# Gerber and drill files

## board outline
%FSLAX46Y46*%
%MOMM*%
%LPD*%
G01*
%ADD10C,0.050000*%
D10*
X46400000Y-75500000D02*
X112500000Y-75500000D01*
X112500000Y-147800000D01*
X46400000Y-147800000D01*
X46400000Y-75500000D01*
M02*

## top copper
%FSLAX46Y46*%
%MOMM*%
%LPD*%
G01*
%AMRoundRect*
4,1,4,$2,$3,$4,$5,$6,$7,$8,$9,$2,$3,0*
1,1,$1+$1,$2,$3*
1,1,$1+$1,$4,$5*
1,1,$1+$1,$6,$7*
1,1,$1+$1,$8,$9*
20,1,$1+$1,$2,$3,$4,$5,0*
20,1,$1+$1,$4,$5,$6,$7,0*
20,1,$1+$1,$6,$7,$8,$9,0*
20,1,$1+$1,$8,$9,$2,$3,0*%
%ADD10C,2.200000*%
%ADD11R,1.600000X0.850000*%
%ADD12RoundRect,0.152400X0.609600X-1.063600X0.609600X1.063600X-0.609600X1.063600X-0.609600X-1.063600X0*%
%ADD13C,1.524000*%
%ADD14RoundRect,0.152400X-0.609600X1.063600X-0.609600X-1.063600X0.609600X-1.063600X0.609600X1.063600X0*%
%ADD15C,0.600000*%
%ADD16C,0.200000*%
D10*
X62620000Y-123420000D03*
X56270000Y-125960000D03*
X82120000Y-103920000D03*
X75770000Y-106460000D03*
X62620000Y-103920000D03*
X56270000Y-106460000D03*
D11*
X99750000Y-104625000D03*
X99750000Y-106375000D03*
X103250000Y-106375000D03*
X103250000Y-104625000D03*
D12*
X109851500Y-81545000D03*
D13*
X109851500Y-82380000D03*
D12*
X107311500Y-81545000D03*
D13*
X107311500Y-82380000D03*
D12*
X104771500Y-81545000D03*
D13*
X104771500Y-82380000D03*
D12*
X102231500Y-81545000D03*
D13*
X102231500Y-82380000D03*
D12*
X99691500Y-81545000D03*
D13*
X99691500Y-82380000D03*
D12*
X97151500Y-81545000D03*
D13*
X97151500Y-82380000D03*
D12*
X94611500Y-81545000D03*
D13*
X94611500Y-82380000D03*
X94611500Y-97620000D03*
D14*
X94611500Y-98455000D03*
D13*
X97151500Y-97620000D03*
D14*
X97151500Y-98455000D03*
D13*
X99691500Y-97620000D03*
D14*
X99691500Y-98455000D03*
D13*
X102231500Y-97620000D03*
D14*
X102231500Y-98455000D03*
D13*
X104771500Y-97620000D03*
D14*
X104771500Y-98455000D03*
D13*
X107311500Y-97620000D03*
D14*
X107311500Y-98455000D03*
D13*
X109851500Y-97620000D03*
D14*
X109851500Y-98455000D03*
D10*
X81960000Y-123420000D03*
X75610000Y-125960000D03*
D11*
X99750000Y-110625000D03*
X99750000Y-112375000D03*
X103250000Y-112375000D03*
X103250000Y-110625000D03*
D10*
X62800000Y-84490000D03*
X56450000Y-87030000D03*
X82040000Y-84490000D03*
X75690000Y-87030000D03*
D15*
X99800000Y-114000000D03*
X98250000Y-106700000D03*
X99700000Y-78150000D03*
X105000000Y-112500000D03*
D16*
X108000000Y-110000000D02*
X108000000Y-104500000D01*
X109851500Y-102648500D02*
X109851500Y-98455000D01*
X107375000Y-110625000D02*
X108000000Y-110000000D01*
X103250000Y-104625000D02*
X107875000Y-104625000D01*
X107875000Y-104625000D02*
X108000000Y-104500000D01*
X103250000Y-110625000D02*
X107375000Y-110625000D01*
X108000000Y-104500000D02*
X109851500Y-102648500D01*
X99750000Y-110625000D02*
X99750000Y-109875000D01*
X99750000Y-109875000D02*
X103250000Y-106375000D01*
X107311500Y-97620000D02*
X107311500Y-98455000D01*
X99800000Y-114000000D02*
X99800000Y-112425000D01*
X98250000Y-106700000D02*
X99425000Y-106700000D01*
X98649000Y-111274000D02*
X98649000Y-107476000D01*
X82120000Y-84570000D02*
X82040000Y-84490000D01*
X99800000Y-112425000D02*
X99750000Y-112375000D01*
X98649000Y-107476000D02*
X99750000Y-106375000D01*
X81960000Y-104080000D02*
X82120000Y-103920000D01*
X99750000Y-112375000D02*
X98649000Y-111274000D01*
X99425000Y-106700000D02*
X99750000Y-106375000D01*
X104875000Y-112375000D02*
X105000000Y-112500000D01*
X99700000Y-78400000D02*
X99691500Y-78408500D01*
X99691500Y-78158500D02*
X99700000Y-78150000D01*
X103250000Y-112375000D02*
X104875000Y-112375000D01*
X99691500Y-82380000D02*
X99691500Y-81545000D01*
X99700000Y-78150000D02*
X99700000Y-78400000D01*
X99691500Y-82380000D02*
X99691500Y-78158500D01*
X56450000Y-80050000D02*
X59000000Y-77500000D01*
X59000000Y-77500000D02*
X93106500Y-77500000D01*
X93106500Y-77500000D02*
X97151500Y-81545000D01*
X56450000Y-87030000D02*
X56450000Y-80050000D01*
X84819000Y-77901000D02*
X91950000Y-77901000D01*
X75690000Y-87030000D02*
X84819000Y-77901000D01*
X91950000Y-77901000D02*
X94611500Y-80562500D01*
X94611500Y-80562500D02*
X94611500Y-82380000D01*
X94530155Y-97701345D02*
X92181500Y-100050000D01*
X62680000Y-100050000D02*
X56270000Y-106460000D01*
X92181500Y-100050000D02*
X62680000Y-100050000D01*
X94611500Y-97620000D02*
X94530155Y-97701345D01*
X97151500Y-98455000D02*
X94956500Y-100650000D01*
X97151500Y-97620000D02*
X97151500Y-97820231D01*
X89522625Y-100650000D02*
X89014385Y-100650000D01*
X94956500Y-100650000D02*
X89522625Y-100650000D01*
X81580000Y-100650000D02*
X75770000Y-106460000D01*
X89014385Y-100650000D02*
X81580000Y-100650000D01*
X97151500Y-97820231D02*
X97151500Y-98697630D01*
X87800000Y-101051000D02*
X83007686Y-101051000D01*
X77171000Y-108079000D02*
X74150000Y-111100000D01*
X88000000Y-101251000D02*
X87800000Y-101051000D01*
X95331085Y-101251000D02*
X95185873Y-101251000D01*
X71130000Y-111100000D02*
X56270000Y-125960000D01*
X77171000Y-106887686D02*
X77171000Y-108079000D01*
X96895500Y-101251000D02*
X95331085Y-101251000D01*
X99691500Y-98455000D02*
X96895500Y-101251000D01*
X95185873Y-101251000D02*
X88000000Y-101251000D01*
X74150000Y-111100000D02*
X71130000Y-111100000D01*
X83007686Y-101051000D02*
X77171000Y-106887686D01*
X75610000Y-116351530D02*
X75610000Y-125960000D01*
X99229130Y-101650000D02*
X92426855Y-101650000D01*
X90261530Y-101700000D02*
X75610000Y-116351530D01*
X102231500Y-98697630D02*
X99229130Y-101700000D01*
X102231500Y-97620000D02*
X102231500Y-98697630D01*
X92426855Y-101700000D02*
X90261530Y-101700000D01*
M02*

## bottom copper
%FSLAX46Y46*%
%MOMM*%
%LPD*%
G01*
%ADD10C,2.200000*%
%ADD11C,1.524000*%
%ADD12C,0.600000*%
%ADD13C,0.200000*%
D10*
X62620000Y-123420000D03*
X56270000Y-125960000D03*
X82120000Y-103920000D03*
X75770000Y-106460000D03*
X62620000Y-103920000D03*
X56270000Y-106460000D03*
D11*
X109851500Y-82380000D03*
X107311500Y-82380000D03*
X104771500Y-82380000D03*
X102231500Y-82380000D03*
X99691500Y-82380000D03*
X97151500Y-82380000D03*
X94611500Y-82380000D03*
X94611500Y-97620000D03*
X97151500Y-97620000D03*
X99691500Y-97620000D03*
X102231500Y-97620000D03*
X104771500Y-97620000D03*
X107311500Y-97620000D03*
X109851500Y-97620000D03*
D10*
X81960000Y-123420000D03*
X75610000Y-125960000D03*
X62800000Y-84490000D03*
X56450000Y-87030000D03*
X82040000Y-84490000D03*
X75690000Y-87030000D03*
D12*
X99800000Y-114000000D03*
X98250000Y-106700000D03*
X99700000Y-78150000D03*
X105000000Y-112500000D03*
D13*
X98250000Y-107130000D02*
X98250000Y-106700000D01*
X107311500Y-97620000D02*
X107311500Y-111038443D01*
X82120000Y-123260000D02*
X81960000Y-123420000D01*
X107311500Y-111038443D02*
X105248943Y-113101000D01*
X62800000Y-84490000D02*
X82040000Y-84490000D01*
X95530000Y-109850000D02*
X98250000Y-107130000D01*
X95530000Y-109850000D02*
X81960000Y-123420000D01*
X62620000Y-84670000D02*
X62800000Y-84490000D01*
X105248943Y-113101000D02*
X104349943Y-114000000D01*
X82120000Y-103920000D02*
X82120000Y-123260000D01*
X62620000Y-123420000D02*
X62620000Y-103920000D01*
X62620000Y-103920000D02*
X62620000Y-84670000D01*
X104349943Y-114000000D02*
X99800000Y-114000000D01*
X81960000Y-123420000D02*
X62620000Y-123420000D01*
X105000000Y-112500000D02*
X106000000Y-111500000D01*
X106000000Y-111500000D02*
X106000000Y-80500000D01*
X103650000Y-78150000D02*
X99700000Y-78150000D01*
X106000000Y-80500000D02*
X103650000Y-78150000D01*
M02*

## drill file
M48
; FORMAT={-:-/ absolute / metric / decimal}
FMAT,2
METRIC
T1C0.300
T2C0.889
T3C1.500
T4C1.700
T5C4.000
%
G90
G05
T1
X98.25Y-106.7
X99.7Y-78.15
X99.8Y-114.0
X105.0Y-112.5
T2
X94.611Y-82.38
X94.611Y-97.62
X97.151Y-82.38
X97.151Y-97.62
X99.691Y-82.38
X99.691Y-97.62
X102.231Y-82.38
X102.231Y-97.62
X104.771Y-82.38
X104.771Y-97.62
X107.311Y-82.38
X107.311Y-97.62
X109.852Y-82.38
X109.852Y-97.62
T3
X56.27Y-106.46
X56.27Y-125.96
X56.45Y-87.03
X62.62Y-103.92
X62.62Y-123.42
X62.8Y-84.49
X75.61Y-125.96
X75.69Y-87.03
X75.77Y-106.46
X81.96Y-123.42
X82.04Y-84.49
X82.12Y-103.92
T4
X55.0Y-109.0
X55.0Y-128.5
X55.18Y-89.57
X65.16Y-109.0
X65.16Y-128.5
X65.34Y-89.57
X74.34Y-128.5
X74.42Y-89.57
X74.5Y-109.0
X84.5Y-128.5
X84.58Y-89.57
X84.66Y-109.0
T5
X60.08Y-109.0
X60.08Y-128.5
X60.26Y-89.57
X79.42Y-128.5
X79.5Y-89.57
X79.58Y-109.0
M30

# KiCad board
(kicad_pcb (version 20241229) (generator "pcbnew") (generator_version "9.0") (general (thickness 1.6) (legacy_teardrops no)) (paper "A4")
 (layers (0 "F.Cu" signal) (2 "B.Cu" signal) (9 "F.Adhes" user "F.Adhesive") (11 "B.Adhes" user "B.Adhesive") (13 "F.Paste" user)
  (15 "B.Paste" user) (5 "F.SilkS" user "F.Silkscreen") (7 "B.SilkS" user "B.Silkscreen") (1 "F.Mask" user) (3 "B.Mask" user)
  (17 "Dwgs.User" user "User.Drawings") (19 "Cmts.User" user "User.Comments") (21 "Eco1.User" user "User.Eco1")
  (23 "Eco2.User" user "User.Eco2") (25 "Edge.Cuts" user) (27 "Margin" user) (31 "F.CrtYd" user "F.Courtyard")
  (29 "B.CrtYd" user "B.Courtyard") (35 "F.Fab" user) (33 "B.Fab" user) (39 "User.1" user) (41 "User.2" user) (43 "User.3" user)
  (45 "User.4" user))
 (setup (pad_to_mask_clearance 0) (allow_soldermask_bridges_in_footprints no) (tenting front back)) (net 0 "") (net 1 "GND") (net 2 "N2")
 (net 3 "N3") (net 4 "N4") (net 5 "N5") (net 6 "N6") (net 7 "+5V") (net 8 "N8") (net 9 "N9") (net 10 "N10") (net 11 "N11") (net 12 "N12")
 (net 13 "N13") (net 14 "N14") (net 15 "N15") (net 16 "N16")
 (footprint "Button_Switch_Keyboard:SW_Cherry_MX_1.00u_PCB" (layer "F.Cu") (at 62.62 123.42)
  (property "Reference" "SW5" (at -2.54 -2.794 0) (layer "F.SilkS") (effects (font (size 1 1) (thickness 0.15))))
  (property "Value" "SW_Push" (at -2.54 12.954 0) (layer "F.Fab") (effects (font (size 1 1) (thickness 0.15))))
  (pad "" np_thru_hole circle (at -7.62 5.08) (size 1.7 1.7) (drill 1.7) (layers "*.Cu" "*.Mask"))
  (pad "" np_thru_hole circle (at -2.54 5.08) (size 4 4) (drill 4) (layers "*.Cu" "*.Mask"))
  (pad "" np_thru_hole circle (at 2.54 5.08) (size 1.7 1.7) (drill 1.7) (layers "*.Cu" "*.Mask"))
  (pad "1" thru_hole circle (at 0 0) (size 2.2 2.2) (drill 1.5) (layers "*.Cu" "*.Mask") (remove_unused_layers no) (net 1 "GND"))
  (pad "2" thru_hole circle (at -6.35 2.54) (size 2.2 2.2) (drill 1.5) (layers "*.Cu" "*.Mask") (remove_unused_layers no) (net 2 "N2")))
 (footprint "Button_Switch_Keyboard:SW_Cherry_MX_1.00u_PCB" (layer "F.Cu") (at 82.12 103.92)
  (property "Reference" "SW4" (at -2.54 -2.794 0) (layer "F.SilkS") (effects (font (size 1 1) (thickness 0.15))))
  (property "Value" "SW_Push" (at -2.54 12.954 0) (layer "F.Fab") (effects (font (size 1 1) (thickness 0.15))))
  (pad "" np_thru_hole circle (at -7.62 5.08) (size 1.7 1.7) (drill 1.7) (layers "*.Cu" "*.Mask"))
  (pad "" np_thru_hole circle (at -2.54 5.08) (size 4 4) (drill 4) (layers "*.Cu" "*.Mask"))
  (pad "" np_thru_hole circle (at 2.54 5.08) (size 1.7 1.7) (drill 1.7) (layers "*.Cu" "*.Mask"))
  (pad "1" thru_hole circle (at 0 0) (size 2.2 2.2) (drill 1.5) (layers "*.Cu" "*.Mask") (remove_unused_layers no) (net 1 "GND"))
  (pad "2" thru_hole circle (at -6.35 2.54) (size 2.2 2.2) (drill 1.5) (layers "*.Cu" "*.Mask") (remove_unused_layers no) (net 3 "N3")))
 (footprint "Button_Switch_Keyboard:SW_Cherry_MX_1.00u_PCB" (layer "F.Cu") (at 62.62 103.92)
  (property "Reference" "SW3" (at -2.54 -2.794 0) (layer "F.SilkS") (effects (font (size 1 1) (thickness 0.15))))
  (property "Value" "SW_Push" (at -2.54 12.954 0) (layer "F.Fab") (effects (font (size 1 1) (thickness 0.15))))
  (pad "" np_thru_hole circle (at -7.62 5.08) (size 1.7 1.7) (drill 1.7) (layers "*.Cu" "*.Mask"))
  (pad "" np_thru_hole circle (at -2.54 5.08) (size 4 4) (drill 4) (layers "*.Cu" "*.Mask"))
  (pad "" np_thru_hole circle (at 2.54 5.08) (size 1.7 1.7) (drill 1.7) (layers "*.Cu" "*.Mask"))
  (pad "1" thru_hole circle (at 0 0) (size 2.2 2.2) (drill 1.5) (layers "*.Cu" "*.Mask") (remove_unused_layers no) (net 1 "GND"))
  (pad "2" thru_hole circle (at -6.35 2.54) (size 2.2 2.2) (drill 1.5) (layers "*.Cu" "*.Mask") (remove_unused_layers no) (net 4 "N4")))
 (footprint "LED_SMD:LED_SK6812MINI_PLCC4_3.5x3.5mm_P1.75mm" (layer "F.Cu") (at 101.5 105.5)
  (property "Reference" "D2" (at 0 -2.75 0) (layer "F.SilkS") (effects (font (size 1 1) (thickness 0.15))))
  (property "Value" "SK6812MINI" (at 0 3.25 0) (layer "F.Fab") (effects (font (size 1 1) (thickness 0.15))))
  (pad "1" smd rect (at -1.75 -0.875) (size 1.6 0.85) (layers "F.Cu" "F.Mask" "F.Paste") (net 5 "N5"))
  (pad "2" smd rect (at -1.75 0.875) (size 1.6 0.85) (layers "F.Cu" "F.Mask" "F.Paste") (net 1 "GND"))
  (pad "3" smd rect (at 1.75 0.875) (size 1.6 0.85) (layers "F.Cu" "F.Mask" "F.Paste") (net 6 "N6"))
  (pad "4" smd rect (at 1.75 -0.875) (size 1.6 0.85) (layers "F.Cu" "F.Mask" "F.Paste") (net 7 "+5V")))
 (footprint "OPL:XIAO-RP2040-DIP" (layer "F.Cu") (at 102.2315 90 -90)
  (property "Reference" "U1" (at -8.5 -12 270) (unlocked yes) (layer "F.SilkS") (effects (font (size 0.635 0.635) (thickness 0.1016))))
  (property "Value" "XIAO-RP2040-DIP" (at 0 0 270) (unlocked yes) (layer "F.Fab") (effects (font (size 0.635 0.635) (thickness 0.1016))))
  (pad "1" smd roundrect (at -8.455 -7.62 90) (size 2.432 1.524) (layers "F.Cu" "F.Mask") (roundrect_rratio 0.1) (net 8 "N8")
   (thermal_bridge_angle 45))
  (pad "1" thru_hole circle (at -7.62 -7.62 90) (size 1.524 1.524) (drill 0.889) (layers "*.Cu" "*.Mask") (remove_unused_layers no)
   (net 8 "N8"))
  (pad "2" smd roundrect (at -8.455 -5.08 90) (size 2.432 1.524) (layers "F.Cu" "F.Mask") (roundrect_rratio 0.1) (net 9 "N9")
   (thermal_bridge_angle 45))
  (pad "2" thru_hole circle (at -7.62 -5.08 90) (size 1.524 1.524) (drill 0.889) (layers "*.Cu" "*.Mask") (remove_unused_layers no)
   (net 9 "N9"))
  (pad "3" smd roundrect (at -8.455 -2.54 90) (size 2.432 1.524) (layers "F.Cu" "F.Mask") (roundrect_rratio 0.1) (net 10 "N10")
   (thermal_bridge_angle 45))
  (pad "3" thru_hole circle (at -7.62 -2.54 90) (size 1.524 1.524) (drill 0.889) (layers "*.Cu" "*.Mask") (remove_unused_layers no)
   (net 10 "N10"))
  (pad "4" smd roundrect (at -8.455 0 90) (size 2.432 1.524) (layers "F.Cu" "F.Mask") (roundrect_rratio 0.1) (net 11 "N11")
   (thermal_bridge_angle 45))
  (pad "4" thru_hole circle (at -7.62 0 90) (size 1.524 1.524) (drill 0.889) (layers "*.Cu" "*.Mask") (remove_unused_layers no)
   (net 11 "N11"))
  (pad "5" smd roundrect (at -8.455 2.54 90) (size 2.432 1.524) (layers "F.Cu" "F.Mask") (roundrect_rratio 0.1) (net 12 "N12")
   (thermal_bridge_angle 45))
  (pad "5" thru_hole circle (at -7.62 2.54 90) (size 1.524 1.524) (drill 0.889) (layers "*.Cu" "*.Mask") (remove_unused_layers no)
   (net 12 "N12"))
  (pad "6" smd roundrect (at -8.455 5.08 90) (size 2.432 1.524) (layers "F.Cu" "F.Mask") (roundrect_rratio 0.1) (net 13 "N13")
   (thermal_bridge_angle 45))
  (pad "6" thru_hole circle (at -7.62 5.08 90) (size 1.524 1.524) (drill 0.889) (layers "*.Cu" "*.Mask") (remove_unused_layers no)
   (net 13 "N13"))
  (pad "7" smd roundrect (at -8.455 7.62 90) (size 2.432 1.524) (layers "F.Cu" "F.Mask") (roundrect_rratio 0.1) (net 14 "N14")
   (thermal_bridge_angle 45))
  (pad "7" thru_hole circle (at -7.62 7.62 90) (size 1.524 1.524) (drill 0.889) (layers "*.Cu" "*.Mask") (remove_unused_layers no)
   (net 14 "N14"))
  (pad "8" thru_hole circle (at 7.62 7.62 270) (size 1.524 1.524) (drill 0.889) (layers "*.Cu" "*.Mask") (remove_unused_layers no)
   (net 4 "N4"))
  (pad "8" smd roundrect (at 8.455 7.62 270) (size 2.432 1.524) (layers "F.Cu" "F.Mask") (roundrect_rratio 0.1) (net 4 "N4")
   (thermal_bridge_angle 45))
  (pad "9" thru_hole circle (at 7.62 5.08 270) (size 1.524 1.524) (drill 0.889) (layers "*.Cu" "*.Mask") (remove_unused_layers no)
   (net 3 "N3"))
  (pad "9" smd roundrect (at 8.455 5.08 270) (size 2.432 1.524) (layers "F.Cu" "F.Mask") (roundrect_rratio 0.1) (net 3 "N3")
   (thermal_bridge_angle 45))
  (pad "10" thru_hole circle (at 7.62 2.54 270) (size 1.524 1.524) (drill 0.889) (layers "*.Cu" "*.Mask") (remove_unused_layers no)
   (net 2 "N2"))
  (pad "10" smd roundrect (at 8.455 2.54 270) (size 2.432 1.524) (layers "F.Cu" "F.Mask") (roundrect_rratio 0.1) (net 2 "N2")
   (thermal_bridge_angle 45))
  (pad "11" thru_hole circle (at 7.62 0 270) (size 1.524 1.524) (drill 0.889) (layers "*.Cu" "*.Mask") (remove_unused_layers no)
   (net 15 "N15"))
  (pad "11" smd roundrect (at 8.455 0 270) (size 2.432 1.524) (layers "F.Cu" "F.Mask") (roundrect_rratio 0.1) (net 15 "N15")
   (thermal_bridge_angle 45))
  (pad "12" thru_hole circle (at 7.62 -2.54 270) (size 1.524 1.524) (drill 0.889) (layers "*.Cu" "*.Mask") (remove_unused_layers no)
   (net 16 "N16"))
  (pad "12" smd roundrect (at 8.455 -2.54 270) (size 2.432 1.524) (layers "F.Cu" "F.Mask") (roundrect_rratio 0.1) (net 16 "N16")
   (thermal_bridge_angle 45))
  (pad "13" thru_hole circle (at 7.62 -5.08 270) (size 1.524 1.524) (drill 0.889) (layers "*.Cu" "*.Mask") (remove_unused_layers no)
   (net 1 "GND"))
  (pad "13" smd roundrect (at 8.455 -5.08 270) (size 2.432 1.524) (layers "F.Cu" "F.Mask") (roundrect_rratio 0.1) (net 1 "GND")
   (thermal_bridge_angle 45))
  (pad "14" thru_hole circle (at 7.62 -7.62 270) (size 1.524 1.524) (drill 0.889) (layers "*.Cu" "*.Mask") (remove_unused_layers no)
   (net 7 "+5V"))
  (pad "14" smd roundrect (at 8.455 -7.62 270) (size 2.432 1.524) (layers "F.Cu" "F.Mask") (roundrect_rratio 0.1) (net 7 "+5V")
   (thermal_bridge_angle 45)))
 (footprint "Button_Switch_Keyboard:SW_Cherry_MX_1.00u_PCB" (layer "F.Cu") (at 81.96 123.42)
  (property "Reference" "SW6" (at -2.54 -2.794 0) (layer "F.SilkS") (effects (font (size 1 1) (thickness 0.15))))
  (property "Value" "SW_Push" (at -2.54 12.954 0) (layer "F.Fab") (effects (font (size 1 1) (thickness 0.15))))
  (pad "" np_thru_hole circle (at -7.62 5.08) (size 1.7 1.7) (drill 1.7) (layers "*.Cu" "*.Mask"))
  (pad "" np_thru_hole circle (at -2.54 5.08) (size 4 4) (drill 4) (layers "*.Cu" "*.Mask"))
  (pad "" np_thru_hole circle (at 2.54 5.08) (size 1.7 1.7) (drill 1.7) (layers "*.Cu" "*.Mask"))
  (pad "1" thru_hole circle (at 0 0) (size 2.2 2.2) (drill 1.5) (layers "*.Cu" "*.Mask") (remove_unused_layers no) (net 1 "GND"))
  (pad "2" thru_hole circle (at -6.35 2.54) (size 2.2 2.2) (drill 1.5) (layers "*.Cu" "*.Mask") (remove_unused_layers no) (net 15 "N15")))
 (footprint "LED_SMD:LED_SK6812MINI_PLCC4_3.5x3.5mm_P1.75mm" (layer "F.Cu") (at 101.5 111.5)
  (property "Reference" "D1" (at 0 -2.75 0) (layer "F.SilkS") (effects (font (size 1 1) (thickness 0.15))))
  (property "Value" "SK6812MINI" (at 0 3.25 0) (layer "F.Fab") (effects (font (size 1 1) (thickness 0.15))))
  (pad "1" smd rect (at -1.75 -0.875) (size 1.6 0.85) (layers "F.Cu" "F.Mask" "F.Paste") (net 6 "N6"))
  (pad "2" smd rect (at -1.75 0.875) (size 1.6 0.85) (layers "F.Cu" "F.Mask" "F.Paste") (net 1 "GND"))
  (pad "3" smd rect (at 1.75 0.875) (size 1.6 0.85) (layers "F.Cu" "F.Mask" "F.Paste") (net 12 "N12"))
  (pad "4" smd rect (at 1.75 -0.875) (size 1.6 0.85) (layers "F.Cu" "F.Mask" "F.Paste") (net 7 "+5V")))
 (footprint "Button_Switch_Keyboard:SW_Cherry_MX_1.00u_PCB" (layer "F.Cu") (at 62.8 84.49)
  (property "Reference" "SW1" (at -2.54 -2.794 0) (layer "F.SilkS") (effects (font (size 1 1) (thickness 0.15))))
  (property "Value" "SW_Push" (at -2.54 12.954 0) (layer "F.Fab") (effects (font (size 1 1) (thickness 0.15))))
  (pad "" np_thru_hole circle (at -7.62 5.08) (size 1.7 1.7) (drill 1.7) (layers "*.Cu" "*.Mask"))
  (pad "" np_thru_hole circle (at -2.54 5.08) (size 4 4) (drill 4) (layers "*.Cu" "*.Mask"))
  (pad "" np_thru_hole circle (at 2.54 5.08) (size 1.7 1.7) (drill 1.7) (layers "*.Cu" "*.Mask"))
  (pad "1" thru_hole circle (at 0 0) (size 2.2 2.2) (drill 1.5) (layers "*.Cu" "*.Mask") (remove_unused_layers no) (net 1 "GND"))
  (pad "2" thru_hole circle (at -6.35 2.54) (size 2.2 2.2) (drill 1.5) (layers "*.Cu" "*.Mask") (remove_unused_layers no) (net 13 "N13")))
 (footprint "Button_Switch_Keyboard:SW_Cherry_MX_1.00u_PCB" (layer "F.Cu") (at 82.04 84.49)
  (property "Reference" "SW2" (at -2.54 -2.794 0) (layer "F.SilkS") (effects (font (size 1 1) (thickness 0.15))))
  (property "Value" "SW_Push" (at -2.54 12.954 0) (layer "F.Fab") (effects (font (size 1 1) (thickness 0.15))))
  (pad "" np_thru_hole circle (at -7.62 5.08) (size 1.7 1.7) (drill 1.7) (layers "*.Cu" "*.Mask"))
  (pad "" np_thru_hole circle (at -2.54 5.08) (size 4 4) (drill 4) (layers "*.Cu" "*.Mask"))
  (pad "" np_thru_hole circle (at 2.54 5.08) (size 1.7 1.7) (drill 1.7) (layers "*.Cu" "*.Mask"))
  (pad "1" thru_hole circle (at 0 0) (size 2.2 2.2) (drill 1.5) (layers "*.Cu" "*.Mask") (remove_unused_layers no) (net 1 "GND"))
  (pad "2" thru_hole circle (at -6.35 2.54) (size 2.2 2.2) (drill 1.5) (layers "*.Cu" "*.Mask") (remove_unused_layers no) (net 14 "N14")))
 (gr_rect (start 46.4 75.5) (end 112.5 147.8) (stroke (width 0.05) (type default)) (fill no) (layer "Edge.Cuts"))
 (segment (start 108 110) (end 108 104.5) (width 0.2) (layer "F.Cu") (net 7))
 (segment (start 109.8515 102.6485) (end 109.8515 98.455) (width 0.2) (layer "F.Cu") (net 7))
 (segment (start 107.375 110.625) (end 108 110) (width 0.2) (layer "F.Cu") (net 7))
 (segment (start 103.25 104.625) (end 107.875 104.625) (width 0.2) (layer "F.Cu") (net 7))
 (segment (start 107.875 104.625) (end 108 104.5) (width 0.2) (layer "F.Cu") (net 7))
 (segment (start 103.25 110.625) (end 107.375 110.625) (width 0.2) (layer "F.Cu") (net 7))
 (segment (start 108 104.5) (end 109.8515 102.6485) (width 0.2) (layer "F.Cu") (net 7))
 (segment (start 99.75 110.625) (end 99.75 109.875) (width 0.2) (layer "F.Cu") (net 6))
 (segment (start 99.75 109.875) (end 103.25 106.375) (width 0.2) (layer "F.Cu") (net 6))
 (segment (start 107.3115 97.62) (end 107.3115 98.455) (width 0.2) (layer "F.Cu") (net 1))
 (segment (start 99.8 114) (end 99.8 112.425) (width 0.2) (layer "F.Cu") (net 1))
 (segment (start 98.25 106.7) (end 99.425 106.7) (width 0.2) (layer "F.Cu") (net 1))
 (segment (start 98.649 111.274) (end 98.649 107.476) (width 0.2) (layer "F.Cu") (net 1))
 (segment (start 82.12 84.57) (end 82.04 84.49) (width 0.2) (layer "F.Cu") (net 1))
 (segment (start 99.8 112.425) (end 99.75 112.375) (width 0.2) (layer "F.Cu") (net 1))
 (segment (start 98.649 107.476) (end 99.75 106.375) (width 0.2) (layer "F.Cu") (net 1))
 (segment (start 81.96 104.08) (end 82.12 103.92) (width 0.2) (layer "F.Cu") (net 1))
 (segment (start 99.75 112.375) (end 98.649 111.274) (width 0.2) (layer "F.Cu") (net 1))
 (segment (start 99.425 106.7) (end 99.75 106.375) (width 0.2) (layer "F.Cu") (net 1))
 (via (at 99.8 114) (size 0.6) (drill 0.3) (layers "F.Cu" "B.Cu") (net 1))
 (via (at 98.25 106.7) (size 0.6) (drill 0.3) (layers "F.Cu" "B.Cu") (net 1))
 (segment (start 98.25 107.13) (end 98.25 106.7) (width 0.2) (layer "B.Cu") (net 1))
 (segment (start 107.3115 97.62) (end 107.3115 111.038443) (width 0.2) (layer "B.Cu") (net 1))
 (segment (start 82.12 123.26) (end 81.96 123.42) (width 0.2) (layer "B.Cu") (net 1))
 (segment (start 107.3115 111.038443) (end 105.248943 113.101) (width 0.2) (layer "B.Cu") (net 1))
 (segment (start 62.8 84.49) (end 82.04 84.49) (width 0.2) (layer "B.Cu") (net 1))
 (segment (start 95.53 109.85) (end 98.25 107.13) (width 0.2) (layer "B.Cu") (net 1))
 (segment (start 95.53 109.85) (end 81.96 123.42) (width 0.2) (layer "B.Cu") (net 1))
 (segment (start 62.62 84.67) (end 62.8 84.49) (width 0.2) (layer "B.Cu") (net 1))
 (segment (start 105.248943 113.101) (end 104.349943 114) (width 0.2) (layer "B.Cu") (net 1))
 (segment (start 82.12 103.92) (end 82.12 123.26) (width 0.2) (layer "B.Cu") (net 1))
 (segment (start 62.62 123.42) (end 62.62 103.92) (width 0.2) (layer "B.Cu") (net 1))
 (segment (start 62.62 103.92) (end 62.62 84.67) (width 0.2) (layer "B.Cu") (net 1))
 (segment (start 104.349943 114) (end 99.8 114) (width 0.2) (layer "B.Cu") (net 1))
 (segment (start 81.96 123.42) (end 62.62 123.42) (width 0.2) (layer "B.Cu") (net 1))
 (segment (start 104.875 112.375) (end 105 112.5) (width 0.2) (layer "F.Cu") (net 12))
 (segment (start 99.7 78.4) (end 99.6915 78.4085) (width 0.2) (layer "F.Cu") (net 12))
 (segment (start 99.6915 78.1585) (end 99.7 78.15) (width 0.2) (layer "F.Cu") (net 12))
 (segment (start 103.25 112.375) (end 104.875 112.375) (width 0.2) (layer "F.Cu") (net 12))
 (segment (start 99.6915 82.38) (end 99.6915 81.545) (width 0.2) (layer "F.Cu") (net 12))
 (segment (start 99.7 78.15) (end 99.7 78.4) (width 0.2) (layer "F.Cu") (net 12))
 (segment (start 99.6915 82.38) (end 99.6915 78.1585) (width 0.2) (layer "F.Cu") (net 12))
 (via (at 99.7 78.15) (size 0.6) (drill 0.3) (layers "F.Cu" "B.Cu") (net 12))
 (via (at 105 112.5) (size 0.6) (drill 0.3) (layers "F.Cu" "B.Cu") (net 12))
 (segment (start 105 112.5) (end 106 111.5) (width 0.2) (layer "B.Cu") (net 12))
 (segment (start 106 111.5) (end 106 80.5) (width 0.2) (layer "B.Cu") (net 12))
 (segment (start 103.65 78.15) (end 99.7 78.15) (width 0.2) (layer "B.Cu") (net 12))
 (segment (start 106 80.5) (end 103.65 78.15) (width 0.2) (layer "B.Cu") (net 12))
 (segment (start 56.45 80.05) (end 59 77.5) (width 0.2) (layer "F.Cu") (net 13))
 (segment (start 59 77.5) (end 93.1065 77.5) (width 0.2) (layer "F.Cu") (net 13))
 (segment (start 93.1065 77.5) (end 97.1515 81.545) (width 0.2) (layer "F.Cu") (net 13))
 (segment (start 56.45 87.03) (end 56.45 80.05) (width 0.2) (layer "F.Cu") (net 13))
 (segment (start 84.819 77.901) (end 91.95 77.901) (width 0.2) (layer "F.Cu") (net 14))
 (segment (start 75.69 87.03) (end 84.819 77.901) (width 0.2) (layer "F.Cu") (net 14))
 (segment (start 91.95 77.901) (end 94.6115 80.5625) (width 0.2) (layer "F.Cu") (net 14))
 (segment (start 94.6115 80.5625) (end 94.6115 82.38) (width 0.2) (layer "F.Cu") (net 14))
 (segment (start 94.530155 97.701345) (end 92.1815 100.05) (width 0.2) (layer "F.Cu") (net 4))
 (segment (start 62.68 100.05) (end 56.27 106.46) (width 0.2) (layer "F.Cu") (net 4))
 (segment (start 92.1815 100.05) (end 62.68 100.05) (width 0.2) (layer "F.Cu") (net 4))
 (segment (start 94.6115 97.62) (end 94.530155 97.701345) (width 0.2) (layer "F.Cu") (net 4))
 (segment (start 97.1515 98.455) (end 94.9565 100.65) (width 0.2) (layer "F.Cu") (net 3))
 (segment (start 97.1515 97.62) (end 97.1515 97.820231) (width 0.2) (layer "F.Cu") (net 3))
 (segment (start 89.522625 100.65) (end 89.014385 100.65) (width 0.2) (layer "F.Cu") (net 3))
 (segment (start 94.9565 100.65) (end 89.522625 100.65) (width 0.2) (layer "F.Cu") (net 3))
 (segment (start 81.58 100.65) (end 75.77 106.46) (width 0.2) (layer "F.Cu") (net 3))
 (segment (start 89.014385 100.65) (end 81.58 100.65) (width 0.2) (layer "F.Cu") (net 3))
 (segment (start 97.1515 97.820231) (end 97.1515 98.69763) (width 0.2) (layer "F.Cu") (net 3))
 (segment (start 87.8 101.051) (end 83.007686 101.051) (width 0.2) (layer "F.Cu") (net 2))
 (segment (start 77.171 108.079) (end 74.15 111.1) (width 0.2) (layer "F.Cu") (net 2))
 (segment (start 88 101.251) (end 87.8 101.051) (width 0.2) (layer "F.Cu") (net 2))
 (segment (start 95.331085 101.251) (end 95.185873 101.251) (width 0.2) (layer "F.Cu") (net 2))
 (segment (start 71.13 111.1) (end 56.27 125.96) (width 0.2) (layer "F.Cu") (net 2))
 (segment (start 77.171 106.887686) (end 77.171 108.079) (width 0.2) (layer "F.Cu") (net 2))
 (segment (start 96.8955 101.251) (end 95.331085 101.251) (width 0.2) (layer "F.Cu") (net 2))
 (segment (start 99.6915 98.455) (end 96.8955 101.251) (width 0.2) (layer "F.Cu") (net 2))
 (segment (start 95.185873 101.251) (end 88 101.251) (width 0.2) (layer "F.Cu") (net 2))
 (segment (start 74.15 111.1) (end 71.13 111.1) (width 0.2) (layer "F.Cu") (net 2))
 (segment (start 83.007686 101.051) (end 77.171 106.887686) (width 0.2) (layer "F.Cu") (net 2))
 (segment (start 75.61 116.35153) (end 75.61 125.96) (width 0.2) (layer "F.Cu") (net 15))
 (segment (start 99.22913 101.65) (end 92.426855 101.65) (width 0.2) (layer "F.Cu") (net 15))
 (segment (start 90.26153 101.7) (end 75.61 116.35153) (width 0.2) (layer "F.Cu") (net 15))
 (segment (start 102.2315 98.69763) (end 99.22913 101.7) (width 0.2) (layer "F.Cu") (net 15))
 (segment (start 102.2315 97.62) (end 102.2315 98.69763) (width 0.2) (layer "F.Cu") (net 15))
 (segment (start 92.426855 101.7) (end 90.26153 101.7) (width 0.2) (layer "F.Cu") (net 15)))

